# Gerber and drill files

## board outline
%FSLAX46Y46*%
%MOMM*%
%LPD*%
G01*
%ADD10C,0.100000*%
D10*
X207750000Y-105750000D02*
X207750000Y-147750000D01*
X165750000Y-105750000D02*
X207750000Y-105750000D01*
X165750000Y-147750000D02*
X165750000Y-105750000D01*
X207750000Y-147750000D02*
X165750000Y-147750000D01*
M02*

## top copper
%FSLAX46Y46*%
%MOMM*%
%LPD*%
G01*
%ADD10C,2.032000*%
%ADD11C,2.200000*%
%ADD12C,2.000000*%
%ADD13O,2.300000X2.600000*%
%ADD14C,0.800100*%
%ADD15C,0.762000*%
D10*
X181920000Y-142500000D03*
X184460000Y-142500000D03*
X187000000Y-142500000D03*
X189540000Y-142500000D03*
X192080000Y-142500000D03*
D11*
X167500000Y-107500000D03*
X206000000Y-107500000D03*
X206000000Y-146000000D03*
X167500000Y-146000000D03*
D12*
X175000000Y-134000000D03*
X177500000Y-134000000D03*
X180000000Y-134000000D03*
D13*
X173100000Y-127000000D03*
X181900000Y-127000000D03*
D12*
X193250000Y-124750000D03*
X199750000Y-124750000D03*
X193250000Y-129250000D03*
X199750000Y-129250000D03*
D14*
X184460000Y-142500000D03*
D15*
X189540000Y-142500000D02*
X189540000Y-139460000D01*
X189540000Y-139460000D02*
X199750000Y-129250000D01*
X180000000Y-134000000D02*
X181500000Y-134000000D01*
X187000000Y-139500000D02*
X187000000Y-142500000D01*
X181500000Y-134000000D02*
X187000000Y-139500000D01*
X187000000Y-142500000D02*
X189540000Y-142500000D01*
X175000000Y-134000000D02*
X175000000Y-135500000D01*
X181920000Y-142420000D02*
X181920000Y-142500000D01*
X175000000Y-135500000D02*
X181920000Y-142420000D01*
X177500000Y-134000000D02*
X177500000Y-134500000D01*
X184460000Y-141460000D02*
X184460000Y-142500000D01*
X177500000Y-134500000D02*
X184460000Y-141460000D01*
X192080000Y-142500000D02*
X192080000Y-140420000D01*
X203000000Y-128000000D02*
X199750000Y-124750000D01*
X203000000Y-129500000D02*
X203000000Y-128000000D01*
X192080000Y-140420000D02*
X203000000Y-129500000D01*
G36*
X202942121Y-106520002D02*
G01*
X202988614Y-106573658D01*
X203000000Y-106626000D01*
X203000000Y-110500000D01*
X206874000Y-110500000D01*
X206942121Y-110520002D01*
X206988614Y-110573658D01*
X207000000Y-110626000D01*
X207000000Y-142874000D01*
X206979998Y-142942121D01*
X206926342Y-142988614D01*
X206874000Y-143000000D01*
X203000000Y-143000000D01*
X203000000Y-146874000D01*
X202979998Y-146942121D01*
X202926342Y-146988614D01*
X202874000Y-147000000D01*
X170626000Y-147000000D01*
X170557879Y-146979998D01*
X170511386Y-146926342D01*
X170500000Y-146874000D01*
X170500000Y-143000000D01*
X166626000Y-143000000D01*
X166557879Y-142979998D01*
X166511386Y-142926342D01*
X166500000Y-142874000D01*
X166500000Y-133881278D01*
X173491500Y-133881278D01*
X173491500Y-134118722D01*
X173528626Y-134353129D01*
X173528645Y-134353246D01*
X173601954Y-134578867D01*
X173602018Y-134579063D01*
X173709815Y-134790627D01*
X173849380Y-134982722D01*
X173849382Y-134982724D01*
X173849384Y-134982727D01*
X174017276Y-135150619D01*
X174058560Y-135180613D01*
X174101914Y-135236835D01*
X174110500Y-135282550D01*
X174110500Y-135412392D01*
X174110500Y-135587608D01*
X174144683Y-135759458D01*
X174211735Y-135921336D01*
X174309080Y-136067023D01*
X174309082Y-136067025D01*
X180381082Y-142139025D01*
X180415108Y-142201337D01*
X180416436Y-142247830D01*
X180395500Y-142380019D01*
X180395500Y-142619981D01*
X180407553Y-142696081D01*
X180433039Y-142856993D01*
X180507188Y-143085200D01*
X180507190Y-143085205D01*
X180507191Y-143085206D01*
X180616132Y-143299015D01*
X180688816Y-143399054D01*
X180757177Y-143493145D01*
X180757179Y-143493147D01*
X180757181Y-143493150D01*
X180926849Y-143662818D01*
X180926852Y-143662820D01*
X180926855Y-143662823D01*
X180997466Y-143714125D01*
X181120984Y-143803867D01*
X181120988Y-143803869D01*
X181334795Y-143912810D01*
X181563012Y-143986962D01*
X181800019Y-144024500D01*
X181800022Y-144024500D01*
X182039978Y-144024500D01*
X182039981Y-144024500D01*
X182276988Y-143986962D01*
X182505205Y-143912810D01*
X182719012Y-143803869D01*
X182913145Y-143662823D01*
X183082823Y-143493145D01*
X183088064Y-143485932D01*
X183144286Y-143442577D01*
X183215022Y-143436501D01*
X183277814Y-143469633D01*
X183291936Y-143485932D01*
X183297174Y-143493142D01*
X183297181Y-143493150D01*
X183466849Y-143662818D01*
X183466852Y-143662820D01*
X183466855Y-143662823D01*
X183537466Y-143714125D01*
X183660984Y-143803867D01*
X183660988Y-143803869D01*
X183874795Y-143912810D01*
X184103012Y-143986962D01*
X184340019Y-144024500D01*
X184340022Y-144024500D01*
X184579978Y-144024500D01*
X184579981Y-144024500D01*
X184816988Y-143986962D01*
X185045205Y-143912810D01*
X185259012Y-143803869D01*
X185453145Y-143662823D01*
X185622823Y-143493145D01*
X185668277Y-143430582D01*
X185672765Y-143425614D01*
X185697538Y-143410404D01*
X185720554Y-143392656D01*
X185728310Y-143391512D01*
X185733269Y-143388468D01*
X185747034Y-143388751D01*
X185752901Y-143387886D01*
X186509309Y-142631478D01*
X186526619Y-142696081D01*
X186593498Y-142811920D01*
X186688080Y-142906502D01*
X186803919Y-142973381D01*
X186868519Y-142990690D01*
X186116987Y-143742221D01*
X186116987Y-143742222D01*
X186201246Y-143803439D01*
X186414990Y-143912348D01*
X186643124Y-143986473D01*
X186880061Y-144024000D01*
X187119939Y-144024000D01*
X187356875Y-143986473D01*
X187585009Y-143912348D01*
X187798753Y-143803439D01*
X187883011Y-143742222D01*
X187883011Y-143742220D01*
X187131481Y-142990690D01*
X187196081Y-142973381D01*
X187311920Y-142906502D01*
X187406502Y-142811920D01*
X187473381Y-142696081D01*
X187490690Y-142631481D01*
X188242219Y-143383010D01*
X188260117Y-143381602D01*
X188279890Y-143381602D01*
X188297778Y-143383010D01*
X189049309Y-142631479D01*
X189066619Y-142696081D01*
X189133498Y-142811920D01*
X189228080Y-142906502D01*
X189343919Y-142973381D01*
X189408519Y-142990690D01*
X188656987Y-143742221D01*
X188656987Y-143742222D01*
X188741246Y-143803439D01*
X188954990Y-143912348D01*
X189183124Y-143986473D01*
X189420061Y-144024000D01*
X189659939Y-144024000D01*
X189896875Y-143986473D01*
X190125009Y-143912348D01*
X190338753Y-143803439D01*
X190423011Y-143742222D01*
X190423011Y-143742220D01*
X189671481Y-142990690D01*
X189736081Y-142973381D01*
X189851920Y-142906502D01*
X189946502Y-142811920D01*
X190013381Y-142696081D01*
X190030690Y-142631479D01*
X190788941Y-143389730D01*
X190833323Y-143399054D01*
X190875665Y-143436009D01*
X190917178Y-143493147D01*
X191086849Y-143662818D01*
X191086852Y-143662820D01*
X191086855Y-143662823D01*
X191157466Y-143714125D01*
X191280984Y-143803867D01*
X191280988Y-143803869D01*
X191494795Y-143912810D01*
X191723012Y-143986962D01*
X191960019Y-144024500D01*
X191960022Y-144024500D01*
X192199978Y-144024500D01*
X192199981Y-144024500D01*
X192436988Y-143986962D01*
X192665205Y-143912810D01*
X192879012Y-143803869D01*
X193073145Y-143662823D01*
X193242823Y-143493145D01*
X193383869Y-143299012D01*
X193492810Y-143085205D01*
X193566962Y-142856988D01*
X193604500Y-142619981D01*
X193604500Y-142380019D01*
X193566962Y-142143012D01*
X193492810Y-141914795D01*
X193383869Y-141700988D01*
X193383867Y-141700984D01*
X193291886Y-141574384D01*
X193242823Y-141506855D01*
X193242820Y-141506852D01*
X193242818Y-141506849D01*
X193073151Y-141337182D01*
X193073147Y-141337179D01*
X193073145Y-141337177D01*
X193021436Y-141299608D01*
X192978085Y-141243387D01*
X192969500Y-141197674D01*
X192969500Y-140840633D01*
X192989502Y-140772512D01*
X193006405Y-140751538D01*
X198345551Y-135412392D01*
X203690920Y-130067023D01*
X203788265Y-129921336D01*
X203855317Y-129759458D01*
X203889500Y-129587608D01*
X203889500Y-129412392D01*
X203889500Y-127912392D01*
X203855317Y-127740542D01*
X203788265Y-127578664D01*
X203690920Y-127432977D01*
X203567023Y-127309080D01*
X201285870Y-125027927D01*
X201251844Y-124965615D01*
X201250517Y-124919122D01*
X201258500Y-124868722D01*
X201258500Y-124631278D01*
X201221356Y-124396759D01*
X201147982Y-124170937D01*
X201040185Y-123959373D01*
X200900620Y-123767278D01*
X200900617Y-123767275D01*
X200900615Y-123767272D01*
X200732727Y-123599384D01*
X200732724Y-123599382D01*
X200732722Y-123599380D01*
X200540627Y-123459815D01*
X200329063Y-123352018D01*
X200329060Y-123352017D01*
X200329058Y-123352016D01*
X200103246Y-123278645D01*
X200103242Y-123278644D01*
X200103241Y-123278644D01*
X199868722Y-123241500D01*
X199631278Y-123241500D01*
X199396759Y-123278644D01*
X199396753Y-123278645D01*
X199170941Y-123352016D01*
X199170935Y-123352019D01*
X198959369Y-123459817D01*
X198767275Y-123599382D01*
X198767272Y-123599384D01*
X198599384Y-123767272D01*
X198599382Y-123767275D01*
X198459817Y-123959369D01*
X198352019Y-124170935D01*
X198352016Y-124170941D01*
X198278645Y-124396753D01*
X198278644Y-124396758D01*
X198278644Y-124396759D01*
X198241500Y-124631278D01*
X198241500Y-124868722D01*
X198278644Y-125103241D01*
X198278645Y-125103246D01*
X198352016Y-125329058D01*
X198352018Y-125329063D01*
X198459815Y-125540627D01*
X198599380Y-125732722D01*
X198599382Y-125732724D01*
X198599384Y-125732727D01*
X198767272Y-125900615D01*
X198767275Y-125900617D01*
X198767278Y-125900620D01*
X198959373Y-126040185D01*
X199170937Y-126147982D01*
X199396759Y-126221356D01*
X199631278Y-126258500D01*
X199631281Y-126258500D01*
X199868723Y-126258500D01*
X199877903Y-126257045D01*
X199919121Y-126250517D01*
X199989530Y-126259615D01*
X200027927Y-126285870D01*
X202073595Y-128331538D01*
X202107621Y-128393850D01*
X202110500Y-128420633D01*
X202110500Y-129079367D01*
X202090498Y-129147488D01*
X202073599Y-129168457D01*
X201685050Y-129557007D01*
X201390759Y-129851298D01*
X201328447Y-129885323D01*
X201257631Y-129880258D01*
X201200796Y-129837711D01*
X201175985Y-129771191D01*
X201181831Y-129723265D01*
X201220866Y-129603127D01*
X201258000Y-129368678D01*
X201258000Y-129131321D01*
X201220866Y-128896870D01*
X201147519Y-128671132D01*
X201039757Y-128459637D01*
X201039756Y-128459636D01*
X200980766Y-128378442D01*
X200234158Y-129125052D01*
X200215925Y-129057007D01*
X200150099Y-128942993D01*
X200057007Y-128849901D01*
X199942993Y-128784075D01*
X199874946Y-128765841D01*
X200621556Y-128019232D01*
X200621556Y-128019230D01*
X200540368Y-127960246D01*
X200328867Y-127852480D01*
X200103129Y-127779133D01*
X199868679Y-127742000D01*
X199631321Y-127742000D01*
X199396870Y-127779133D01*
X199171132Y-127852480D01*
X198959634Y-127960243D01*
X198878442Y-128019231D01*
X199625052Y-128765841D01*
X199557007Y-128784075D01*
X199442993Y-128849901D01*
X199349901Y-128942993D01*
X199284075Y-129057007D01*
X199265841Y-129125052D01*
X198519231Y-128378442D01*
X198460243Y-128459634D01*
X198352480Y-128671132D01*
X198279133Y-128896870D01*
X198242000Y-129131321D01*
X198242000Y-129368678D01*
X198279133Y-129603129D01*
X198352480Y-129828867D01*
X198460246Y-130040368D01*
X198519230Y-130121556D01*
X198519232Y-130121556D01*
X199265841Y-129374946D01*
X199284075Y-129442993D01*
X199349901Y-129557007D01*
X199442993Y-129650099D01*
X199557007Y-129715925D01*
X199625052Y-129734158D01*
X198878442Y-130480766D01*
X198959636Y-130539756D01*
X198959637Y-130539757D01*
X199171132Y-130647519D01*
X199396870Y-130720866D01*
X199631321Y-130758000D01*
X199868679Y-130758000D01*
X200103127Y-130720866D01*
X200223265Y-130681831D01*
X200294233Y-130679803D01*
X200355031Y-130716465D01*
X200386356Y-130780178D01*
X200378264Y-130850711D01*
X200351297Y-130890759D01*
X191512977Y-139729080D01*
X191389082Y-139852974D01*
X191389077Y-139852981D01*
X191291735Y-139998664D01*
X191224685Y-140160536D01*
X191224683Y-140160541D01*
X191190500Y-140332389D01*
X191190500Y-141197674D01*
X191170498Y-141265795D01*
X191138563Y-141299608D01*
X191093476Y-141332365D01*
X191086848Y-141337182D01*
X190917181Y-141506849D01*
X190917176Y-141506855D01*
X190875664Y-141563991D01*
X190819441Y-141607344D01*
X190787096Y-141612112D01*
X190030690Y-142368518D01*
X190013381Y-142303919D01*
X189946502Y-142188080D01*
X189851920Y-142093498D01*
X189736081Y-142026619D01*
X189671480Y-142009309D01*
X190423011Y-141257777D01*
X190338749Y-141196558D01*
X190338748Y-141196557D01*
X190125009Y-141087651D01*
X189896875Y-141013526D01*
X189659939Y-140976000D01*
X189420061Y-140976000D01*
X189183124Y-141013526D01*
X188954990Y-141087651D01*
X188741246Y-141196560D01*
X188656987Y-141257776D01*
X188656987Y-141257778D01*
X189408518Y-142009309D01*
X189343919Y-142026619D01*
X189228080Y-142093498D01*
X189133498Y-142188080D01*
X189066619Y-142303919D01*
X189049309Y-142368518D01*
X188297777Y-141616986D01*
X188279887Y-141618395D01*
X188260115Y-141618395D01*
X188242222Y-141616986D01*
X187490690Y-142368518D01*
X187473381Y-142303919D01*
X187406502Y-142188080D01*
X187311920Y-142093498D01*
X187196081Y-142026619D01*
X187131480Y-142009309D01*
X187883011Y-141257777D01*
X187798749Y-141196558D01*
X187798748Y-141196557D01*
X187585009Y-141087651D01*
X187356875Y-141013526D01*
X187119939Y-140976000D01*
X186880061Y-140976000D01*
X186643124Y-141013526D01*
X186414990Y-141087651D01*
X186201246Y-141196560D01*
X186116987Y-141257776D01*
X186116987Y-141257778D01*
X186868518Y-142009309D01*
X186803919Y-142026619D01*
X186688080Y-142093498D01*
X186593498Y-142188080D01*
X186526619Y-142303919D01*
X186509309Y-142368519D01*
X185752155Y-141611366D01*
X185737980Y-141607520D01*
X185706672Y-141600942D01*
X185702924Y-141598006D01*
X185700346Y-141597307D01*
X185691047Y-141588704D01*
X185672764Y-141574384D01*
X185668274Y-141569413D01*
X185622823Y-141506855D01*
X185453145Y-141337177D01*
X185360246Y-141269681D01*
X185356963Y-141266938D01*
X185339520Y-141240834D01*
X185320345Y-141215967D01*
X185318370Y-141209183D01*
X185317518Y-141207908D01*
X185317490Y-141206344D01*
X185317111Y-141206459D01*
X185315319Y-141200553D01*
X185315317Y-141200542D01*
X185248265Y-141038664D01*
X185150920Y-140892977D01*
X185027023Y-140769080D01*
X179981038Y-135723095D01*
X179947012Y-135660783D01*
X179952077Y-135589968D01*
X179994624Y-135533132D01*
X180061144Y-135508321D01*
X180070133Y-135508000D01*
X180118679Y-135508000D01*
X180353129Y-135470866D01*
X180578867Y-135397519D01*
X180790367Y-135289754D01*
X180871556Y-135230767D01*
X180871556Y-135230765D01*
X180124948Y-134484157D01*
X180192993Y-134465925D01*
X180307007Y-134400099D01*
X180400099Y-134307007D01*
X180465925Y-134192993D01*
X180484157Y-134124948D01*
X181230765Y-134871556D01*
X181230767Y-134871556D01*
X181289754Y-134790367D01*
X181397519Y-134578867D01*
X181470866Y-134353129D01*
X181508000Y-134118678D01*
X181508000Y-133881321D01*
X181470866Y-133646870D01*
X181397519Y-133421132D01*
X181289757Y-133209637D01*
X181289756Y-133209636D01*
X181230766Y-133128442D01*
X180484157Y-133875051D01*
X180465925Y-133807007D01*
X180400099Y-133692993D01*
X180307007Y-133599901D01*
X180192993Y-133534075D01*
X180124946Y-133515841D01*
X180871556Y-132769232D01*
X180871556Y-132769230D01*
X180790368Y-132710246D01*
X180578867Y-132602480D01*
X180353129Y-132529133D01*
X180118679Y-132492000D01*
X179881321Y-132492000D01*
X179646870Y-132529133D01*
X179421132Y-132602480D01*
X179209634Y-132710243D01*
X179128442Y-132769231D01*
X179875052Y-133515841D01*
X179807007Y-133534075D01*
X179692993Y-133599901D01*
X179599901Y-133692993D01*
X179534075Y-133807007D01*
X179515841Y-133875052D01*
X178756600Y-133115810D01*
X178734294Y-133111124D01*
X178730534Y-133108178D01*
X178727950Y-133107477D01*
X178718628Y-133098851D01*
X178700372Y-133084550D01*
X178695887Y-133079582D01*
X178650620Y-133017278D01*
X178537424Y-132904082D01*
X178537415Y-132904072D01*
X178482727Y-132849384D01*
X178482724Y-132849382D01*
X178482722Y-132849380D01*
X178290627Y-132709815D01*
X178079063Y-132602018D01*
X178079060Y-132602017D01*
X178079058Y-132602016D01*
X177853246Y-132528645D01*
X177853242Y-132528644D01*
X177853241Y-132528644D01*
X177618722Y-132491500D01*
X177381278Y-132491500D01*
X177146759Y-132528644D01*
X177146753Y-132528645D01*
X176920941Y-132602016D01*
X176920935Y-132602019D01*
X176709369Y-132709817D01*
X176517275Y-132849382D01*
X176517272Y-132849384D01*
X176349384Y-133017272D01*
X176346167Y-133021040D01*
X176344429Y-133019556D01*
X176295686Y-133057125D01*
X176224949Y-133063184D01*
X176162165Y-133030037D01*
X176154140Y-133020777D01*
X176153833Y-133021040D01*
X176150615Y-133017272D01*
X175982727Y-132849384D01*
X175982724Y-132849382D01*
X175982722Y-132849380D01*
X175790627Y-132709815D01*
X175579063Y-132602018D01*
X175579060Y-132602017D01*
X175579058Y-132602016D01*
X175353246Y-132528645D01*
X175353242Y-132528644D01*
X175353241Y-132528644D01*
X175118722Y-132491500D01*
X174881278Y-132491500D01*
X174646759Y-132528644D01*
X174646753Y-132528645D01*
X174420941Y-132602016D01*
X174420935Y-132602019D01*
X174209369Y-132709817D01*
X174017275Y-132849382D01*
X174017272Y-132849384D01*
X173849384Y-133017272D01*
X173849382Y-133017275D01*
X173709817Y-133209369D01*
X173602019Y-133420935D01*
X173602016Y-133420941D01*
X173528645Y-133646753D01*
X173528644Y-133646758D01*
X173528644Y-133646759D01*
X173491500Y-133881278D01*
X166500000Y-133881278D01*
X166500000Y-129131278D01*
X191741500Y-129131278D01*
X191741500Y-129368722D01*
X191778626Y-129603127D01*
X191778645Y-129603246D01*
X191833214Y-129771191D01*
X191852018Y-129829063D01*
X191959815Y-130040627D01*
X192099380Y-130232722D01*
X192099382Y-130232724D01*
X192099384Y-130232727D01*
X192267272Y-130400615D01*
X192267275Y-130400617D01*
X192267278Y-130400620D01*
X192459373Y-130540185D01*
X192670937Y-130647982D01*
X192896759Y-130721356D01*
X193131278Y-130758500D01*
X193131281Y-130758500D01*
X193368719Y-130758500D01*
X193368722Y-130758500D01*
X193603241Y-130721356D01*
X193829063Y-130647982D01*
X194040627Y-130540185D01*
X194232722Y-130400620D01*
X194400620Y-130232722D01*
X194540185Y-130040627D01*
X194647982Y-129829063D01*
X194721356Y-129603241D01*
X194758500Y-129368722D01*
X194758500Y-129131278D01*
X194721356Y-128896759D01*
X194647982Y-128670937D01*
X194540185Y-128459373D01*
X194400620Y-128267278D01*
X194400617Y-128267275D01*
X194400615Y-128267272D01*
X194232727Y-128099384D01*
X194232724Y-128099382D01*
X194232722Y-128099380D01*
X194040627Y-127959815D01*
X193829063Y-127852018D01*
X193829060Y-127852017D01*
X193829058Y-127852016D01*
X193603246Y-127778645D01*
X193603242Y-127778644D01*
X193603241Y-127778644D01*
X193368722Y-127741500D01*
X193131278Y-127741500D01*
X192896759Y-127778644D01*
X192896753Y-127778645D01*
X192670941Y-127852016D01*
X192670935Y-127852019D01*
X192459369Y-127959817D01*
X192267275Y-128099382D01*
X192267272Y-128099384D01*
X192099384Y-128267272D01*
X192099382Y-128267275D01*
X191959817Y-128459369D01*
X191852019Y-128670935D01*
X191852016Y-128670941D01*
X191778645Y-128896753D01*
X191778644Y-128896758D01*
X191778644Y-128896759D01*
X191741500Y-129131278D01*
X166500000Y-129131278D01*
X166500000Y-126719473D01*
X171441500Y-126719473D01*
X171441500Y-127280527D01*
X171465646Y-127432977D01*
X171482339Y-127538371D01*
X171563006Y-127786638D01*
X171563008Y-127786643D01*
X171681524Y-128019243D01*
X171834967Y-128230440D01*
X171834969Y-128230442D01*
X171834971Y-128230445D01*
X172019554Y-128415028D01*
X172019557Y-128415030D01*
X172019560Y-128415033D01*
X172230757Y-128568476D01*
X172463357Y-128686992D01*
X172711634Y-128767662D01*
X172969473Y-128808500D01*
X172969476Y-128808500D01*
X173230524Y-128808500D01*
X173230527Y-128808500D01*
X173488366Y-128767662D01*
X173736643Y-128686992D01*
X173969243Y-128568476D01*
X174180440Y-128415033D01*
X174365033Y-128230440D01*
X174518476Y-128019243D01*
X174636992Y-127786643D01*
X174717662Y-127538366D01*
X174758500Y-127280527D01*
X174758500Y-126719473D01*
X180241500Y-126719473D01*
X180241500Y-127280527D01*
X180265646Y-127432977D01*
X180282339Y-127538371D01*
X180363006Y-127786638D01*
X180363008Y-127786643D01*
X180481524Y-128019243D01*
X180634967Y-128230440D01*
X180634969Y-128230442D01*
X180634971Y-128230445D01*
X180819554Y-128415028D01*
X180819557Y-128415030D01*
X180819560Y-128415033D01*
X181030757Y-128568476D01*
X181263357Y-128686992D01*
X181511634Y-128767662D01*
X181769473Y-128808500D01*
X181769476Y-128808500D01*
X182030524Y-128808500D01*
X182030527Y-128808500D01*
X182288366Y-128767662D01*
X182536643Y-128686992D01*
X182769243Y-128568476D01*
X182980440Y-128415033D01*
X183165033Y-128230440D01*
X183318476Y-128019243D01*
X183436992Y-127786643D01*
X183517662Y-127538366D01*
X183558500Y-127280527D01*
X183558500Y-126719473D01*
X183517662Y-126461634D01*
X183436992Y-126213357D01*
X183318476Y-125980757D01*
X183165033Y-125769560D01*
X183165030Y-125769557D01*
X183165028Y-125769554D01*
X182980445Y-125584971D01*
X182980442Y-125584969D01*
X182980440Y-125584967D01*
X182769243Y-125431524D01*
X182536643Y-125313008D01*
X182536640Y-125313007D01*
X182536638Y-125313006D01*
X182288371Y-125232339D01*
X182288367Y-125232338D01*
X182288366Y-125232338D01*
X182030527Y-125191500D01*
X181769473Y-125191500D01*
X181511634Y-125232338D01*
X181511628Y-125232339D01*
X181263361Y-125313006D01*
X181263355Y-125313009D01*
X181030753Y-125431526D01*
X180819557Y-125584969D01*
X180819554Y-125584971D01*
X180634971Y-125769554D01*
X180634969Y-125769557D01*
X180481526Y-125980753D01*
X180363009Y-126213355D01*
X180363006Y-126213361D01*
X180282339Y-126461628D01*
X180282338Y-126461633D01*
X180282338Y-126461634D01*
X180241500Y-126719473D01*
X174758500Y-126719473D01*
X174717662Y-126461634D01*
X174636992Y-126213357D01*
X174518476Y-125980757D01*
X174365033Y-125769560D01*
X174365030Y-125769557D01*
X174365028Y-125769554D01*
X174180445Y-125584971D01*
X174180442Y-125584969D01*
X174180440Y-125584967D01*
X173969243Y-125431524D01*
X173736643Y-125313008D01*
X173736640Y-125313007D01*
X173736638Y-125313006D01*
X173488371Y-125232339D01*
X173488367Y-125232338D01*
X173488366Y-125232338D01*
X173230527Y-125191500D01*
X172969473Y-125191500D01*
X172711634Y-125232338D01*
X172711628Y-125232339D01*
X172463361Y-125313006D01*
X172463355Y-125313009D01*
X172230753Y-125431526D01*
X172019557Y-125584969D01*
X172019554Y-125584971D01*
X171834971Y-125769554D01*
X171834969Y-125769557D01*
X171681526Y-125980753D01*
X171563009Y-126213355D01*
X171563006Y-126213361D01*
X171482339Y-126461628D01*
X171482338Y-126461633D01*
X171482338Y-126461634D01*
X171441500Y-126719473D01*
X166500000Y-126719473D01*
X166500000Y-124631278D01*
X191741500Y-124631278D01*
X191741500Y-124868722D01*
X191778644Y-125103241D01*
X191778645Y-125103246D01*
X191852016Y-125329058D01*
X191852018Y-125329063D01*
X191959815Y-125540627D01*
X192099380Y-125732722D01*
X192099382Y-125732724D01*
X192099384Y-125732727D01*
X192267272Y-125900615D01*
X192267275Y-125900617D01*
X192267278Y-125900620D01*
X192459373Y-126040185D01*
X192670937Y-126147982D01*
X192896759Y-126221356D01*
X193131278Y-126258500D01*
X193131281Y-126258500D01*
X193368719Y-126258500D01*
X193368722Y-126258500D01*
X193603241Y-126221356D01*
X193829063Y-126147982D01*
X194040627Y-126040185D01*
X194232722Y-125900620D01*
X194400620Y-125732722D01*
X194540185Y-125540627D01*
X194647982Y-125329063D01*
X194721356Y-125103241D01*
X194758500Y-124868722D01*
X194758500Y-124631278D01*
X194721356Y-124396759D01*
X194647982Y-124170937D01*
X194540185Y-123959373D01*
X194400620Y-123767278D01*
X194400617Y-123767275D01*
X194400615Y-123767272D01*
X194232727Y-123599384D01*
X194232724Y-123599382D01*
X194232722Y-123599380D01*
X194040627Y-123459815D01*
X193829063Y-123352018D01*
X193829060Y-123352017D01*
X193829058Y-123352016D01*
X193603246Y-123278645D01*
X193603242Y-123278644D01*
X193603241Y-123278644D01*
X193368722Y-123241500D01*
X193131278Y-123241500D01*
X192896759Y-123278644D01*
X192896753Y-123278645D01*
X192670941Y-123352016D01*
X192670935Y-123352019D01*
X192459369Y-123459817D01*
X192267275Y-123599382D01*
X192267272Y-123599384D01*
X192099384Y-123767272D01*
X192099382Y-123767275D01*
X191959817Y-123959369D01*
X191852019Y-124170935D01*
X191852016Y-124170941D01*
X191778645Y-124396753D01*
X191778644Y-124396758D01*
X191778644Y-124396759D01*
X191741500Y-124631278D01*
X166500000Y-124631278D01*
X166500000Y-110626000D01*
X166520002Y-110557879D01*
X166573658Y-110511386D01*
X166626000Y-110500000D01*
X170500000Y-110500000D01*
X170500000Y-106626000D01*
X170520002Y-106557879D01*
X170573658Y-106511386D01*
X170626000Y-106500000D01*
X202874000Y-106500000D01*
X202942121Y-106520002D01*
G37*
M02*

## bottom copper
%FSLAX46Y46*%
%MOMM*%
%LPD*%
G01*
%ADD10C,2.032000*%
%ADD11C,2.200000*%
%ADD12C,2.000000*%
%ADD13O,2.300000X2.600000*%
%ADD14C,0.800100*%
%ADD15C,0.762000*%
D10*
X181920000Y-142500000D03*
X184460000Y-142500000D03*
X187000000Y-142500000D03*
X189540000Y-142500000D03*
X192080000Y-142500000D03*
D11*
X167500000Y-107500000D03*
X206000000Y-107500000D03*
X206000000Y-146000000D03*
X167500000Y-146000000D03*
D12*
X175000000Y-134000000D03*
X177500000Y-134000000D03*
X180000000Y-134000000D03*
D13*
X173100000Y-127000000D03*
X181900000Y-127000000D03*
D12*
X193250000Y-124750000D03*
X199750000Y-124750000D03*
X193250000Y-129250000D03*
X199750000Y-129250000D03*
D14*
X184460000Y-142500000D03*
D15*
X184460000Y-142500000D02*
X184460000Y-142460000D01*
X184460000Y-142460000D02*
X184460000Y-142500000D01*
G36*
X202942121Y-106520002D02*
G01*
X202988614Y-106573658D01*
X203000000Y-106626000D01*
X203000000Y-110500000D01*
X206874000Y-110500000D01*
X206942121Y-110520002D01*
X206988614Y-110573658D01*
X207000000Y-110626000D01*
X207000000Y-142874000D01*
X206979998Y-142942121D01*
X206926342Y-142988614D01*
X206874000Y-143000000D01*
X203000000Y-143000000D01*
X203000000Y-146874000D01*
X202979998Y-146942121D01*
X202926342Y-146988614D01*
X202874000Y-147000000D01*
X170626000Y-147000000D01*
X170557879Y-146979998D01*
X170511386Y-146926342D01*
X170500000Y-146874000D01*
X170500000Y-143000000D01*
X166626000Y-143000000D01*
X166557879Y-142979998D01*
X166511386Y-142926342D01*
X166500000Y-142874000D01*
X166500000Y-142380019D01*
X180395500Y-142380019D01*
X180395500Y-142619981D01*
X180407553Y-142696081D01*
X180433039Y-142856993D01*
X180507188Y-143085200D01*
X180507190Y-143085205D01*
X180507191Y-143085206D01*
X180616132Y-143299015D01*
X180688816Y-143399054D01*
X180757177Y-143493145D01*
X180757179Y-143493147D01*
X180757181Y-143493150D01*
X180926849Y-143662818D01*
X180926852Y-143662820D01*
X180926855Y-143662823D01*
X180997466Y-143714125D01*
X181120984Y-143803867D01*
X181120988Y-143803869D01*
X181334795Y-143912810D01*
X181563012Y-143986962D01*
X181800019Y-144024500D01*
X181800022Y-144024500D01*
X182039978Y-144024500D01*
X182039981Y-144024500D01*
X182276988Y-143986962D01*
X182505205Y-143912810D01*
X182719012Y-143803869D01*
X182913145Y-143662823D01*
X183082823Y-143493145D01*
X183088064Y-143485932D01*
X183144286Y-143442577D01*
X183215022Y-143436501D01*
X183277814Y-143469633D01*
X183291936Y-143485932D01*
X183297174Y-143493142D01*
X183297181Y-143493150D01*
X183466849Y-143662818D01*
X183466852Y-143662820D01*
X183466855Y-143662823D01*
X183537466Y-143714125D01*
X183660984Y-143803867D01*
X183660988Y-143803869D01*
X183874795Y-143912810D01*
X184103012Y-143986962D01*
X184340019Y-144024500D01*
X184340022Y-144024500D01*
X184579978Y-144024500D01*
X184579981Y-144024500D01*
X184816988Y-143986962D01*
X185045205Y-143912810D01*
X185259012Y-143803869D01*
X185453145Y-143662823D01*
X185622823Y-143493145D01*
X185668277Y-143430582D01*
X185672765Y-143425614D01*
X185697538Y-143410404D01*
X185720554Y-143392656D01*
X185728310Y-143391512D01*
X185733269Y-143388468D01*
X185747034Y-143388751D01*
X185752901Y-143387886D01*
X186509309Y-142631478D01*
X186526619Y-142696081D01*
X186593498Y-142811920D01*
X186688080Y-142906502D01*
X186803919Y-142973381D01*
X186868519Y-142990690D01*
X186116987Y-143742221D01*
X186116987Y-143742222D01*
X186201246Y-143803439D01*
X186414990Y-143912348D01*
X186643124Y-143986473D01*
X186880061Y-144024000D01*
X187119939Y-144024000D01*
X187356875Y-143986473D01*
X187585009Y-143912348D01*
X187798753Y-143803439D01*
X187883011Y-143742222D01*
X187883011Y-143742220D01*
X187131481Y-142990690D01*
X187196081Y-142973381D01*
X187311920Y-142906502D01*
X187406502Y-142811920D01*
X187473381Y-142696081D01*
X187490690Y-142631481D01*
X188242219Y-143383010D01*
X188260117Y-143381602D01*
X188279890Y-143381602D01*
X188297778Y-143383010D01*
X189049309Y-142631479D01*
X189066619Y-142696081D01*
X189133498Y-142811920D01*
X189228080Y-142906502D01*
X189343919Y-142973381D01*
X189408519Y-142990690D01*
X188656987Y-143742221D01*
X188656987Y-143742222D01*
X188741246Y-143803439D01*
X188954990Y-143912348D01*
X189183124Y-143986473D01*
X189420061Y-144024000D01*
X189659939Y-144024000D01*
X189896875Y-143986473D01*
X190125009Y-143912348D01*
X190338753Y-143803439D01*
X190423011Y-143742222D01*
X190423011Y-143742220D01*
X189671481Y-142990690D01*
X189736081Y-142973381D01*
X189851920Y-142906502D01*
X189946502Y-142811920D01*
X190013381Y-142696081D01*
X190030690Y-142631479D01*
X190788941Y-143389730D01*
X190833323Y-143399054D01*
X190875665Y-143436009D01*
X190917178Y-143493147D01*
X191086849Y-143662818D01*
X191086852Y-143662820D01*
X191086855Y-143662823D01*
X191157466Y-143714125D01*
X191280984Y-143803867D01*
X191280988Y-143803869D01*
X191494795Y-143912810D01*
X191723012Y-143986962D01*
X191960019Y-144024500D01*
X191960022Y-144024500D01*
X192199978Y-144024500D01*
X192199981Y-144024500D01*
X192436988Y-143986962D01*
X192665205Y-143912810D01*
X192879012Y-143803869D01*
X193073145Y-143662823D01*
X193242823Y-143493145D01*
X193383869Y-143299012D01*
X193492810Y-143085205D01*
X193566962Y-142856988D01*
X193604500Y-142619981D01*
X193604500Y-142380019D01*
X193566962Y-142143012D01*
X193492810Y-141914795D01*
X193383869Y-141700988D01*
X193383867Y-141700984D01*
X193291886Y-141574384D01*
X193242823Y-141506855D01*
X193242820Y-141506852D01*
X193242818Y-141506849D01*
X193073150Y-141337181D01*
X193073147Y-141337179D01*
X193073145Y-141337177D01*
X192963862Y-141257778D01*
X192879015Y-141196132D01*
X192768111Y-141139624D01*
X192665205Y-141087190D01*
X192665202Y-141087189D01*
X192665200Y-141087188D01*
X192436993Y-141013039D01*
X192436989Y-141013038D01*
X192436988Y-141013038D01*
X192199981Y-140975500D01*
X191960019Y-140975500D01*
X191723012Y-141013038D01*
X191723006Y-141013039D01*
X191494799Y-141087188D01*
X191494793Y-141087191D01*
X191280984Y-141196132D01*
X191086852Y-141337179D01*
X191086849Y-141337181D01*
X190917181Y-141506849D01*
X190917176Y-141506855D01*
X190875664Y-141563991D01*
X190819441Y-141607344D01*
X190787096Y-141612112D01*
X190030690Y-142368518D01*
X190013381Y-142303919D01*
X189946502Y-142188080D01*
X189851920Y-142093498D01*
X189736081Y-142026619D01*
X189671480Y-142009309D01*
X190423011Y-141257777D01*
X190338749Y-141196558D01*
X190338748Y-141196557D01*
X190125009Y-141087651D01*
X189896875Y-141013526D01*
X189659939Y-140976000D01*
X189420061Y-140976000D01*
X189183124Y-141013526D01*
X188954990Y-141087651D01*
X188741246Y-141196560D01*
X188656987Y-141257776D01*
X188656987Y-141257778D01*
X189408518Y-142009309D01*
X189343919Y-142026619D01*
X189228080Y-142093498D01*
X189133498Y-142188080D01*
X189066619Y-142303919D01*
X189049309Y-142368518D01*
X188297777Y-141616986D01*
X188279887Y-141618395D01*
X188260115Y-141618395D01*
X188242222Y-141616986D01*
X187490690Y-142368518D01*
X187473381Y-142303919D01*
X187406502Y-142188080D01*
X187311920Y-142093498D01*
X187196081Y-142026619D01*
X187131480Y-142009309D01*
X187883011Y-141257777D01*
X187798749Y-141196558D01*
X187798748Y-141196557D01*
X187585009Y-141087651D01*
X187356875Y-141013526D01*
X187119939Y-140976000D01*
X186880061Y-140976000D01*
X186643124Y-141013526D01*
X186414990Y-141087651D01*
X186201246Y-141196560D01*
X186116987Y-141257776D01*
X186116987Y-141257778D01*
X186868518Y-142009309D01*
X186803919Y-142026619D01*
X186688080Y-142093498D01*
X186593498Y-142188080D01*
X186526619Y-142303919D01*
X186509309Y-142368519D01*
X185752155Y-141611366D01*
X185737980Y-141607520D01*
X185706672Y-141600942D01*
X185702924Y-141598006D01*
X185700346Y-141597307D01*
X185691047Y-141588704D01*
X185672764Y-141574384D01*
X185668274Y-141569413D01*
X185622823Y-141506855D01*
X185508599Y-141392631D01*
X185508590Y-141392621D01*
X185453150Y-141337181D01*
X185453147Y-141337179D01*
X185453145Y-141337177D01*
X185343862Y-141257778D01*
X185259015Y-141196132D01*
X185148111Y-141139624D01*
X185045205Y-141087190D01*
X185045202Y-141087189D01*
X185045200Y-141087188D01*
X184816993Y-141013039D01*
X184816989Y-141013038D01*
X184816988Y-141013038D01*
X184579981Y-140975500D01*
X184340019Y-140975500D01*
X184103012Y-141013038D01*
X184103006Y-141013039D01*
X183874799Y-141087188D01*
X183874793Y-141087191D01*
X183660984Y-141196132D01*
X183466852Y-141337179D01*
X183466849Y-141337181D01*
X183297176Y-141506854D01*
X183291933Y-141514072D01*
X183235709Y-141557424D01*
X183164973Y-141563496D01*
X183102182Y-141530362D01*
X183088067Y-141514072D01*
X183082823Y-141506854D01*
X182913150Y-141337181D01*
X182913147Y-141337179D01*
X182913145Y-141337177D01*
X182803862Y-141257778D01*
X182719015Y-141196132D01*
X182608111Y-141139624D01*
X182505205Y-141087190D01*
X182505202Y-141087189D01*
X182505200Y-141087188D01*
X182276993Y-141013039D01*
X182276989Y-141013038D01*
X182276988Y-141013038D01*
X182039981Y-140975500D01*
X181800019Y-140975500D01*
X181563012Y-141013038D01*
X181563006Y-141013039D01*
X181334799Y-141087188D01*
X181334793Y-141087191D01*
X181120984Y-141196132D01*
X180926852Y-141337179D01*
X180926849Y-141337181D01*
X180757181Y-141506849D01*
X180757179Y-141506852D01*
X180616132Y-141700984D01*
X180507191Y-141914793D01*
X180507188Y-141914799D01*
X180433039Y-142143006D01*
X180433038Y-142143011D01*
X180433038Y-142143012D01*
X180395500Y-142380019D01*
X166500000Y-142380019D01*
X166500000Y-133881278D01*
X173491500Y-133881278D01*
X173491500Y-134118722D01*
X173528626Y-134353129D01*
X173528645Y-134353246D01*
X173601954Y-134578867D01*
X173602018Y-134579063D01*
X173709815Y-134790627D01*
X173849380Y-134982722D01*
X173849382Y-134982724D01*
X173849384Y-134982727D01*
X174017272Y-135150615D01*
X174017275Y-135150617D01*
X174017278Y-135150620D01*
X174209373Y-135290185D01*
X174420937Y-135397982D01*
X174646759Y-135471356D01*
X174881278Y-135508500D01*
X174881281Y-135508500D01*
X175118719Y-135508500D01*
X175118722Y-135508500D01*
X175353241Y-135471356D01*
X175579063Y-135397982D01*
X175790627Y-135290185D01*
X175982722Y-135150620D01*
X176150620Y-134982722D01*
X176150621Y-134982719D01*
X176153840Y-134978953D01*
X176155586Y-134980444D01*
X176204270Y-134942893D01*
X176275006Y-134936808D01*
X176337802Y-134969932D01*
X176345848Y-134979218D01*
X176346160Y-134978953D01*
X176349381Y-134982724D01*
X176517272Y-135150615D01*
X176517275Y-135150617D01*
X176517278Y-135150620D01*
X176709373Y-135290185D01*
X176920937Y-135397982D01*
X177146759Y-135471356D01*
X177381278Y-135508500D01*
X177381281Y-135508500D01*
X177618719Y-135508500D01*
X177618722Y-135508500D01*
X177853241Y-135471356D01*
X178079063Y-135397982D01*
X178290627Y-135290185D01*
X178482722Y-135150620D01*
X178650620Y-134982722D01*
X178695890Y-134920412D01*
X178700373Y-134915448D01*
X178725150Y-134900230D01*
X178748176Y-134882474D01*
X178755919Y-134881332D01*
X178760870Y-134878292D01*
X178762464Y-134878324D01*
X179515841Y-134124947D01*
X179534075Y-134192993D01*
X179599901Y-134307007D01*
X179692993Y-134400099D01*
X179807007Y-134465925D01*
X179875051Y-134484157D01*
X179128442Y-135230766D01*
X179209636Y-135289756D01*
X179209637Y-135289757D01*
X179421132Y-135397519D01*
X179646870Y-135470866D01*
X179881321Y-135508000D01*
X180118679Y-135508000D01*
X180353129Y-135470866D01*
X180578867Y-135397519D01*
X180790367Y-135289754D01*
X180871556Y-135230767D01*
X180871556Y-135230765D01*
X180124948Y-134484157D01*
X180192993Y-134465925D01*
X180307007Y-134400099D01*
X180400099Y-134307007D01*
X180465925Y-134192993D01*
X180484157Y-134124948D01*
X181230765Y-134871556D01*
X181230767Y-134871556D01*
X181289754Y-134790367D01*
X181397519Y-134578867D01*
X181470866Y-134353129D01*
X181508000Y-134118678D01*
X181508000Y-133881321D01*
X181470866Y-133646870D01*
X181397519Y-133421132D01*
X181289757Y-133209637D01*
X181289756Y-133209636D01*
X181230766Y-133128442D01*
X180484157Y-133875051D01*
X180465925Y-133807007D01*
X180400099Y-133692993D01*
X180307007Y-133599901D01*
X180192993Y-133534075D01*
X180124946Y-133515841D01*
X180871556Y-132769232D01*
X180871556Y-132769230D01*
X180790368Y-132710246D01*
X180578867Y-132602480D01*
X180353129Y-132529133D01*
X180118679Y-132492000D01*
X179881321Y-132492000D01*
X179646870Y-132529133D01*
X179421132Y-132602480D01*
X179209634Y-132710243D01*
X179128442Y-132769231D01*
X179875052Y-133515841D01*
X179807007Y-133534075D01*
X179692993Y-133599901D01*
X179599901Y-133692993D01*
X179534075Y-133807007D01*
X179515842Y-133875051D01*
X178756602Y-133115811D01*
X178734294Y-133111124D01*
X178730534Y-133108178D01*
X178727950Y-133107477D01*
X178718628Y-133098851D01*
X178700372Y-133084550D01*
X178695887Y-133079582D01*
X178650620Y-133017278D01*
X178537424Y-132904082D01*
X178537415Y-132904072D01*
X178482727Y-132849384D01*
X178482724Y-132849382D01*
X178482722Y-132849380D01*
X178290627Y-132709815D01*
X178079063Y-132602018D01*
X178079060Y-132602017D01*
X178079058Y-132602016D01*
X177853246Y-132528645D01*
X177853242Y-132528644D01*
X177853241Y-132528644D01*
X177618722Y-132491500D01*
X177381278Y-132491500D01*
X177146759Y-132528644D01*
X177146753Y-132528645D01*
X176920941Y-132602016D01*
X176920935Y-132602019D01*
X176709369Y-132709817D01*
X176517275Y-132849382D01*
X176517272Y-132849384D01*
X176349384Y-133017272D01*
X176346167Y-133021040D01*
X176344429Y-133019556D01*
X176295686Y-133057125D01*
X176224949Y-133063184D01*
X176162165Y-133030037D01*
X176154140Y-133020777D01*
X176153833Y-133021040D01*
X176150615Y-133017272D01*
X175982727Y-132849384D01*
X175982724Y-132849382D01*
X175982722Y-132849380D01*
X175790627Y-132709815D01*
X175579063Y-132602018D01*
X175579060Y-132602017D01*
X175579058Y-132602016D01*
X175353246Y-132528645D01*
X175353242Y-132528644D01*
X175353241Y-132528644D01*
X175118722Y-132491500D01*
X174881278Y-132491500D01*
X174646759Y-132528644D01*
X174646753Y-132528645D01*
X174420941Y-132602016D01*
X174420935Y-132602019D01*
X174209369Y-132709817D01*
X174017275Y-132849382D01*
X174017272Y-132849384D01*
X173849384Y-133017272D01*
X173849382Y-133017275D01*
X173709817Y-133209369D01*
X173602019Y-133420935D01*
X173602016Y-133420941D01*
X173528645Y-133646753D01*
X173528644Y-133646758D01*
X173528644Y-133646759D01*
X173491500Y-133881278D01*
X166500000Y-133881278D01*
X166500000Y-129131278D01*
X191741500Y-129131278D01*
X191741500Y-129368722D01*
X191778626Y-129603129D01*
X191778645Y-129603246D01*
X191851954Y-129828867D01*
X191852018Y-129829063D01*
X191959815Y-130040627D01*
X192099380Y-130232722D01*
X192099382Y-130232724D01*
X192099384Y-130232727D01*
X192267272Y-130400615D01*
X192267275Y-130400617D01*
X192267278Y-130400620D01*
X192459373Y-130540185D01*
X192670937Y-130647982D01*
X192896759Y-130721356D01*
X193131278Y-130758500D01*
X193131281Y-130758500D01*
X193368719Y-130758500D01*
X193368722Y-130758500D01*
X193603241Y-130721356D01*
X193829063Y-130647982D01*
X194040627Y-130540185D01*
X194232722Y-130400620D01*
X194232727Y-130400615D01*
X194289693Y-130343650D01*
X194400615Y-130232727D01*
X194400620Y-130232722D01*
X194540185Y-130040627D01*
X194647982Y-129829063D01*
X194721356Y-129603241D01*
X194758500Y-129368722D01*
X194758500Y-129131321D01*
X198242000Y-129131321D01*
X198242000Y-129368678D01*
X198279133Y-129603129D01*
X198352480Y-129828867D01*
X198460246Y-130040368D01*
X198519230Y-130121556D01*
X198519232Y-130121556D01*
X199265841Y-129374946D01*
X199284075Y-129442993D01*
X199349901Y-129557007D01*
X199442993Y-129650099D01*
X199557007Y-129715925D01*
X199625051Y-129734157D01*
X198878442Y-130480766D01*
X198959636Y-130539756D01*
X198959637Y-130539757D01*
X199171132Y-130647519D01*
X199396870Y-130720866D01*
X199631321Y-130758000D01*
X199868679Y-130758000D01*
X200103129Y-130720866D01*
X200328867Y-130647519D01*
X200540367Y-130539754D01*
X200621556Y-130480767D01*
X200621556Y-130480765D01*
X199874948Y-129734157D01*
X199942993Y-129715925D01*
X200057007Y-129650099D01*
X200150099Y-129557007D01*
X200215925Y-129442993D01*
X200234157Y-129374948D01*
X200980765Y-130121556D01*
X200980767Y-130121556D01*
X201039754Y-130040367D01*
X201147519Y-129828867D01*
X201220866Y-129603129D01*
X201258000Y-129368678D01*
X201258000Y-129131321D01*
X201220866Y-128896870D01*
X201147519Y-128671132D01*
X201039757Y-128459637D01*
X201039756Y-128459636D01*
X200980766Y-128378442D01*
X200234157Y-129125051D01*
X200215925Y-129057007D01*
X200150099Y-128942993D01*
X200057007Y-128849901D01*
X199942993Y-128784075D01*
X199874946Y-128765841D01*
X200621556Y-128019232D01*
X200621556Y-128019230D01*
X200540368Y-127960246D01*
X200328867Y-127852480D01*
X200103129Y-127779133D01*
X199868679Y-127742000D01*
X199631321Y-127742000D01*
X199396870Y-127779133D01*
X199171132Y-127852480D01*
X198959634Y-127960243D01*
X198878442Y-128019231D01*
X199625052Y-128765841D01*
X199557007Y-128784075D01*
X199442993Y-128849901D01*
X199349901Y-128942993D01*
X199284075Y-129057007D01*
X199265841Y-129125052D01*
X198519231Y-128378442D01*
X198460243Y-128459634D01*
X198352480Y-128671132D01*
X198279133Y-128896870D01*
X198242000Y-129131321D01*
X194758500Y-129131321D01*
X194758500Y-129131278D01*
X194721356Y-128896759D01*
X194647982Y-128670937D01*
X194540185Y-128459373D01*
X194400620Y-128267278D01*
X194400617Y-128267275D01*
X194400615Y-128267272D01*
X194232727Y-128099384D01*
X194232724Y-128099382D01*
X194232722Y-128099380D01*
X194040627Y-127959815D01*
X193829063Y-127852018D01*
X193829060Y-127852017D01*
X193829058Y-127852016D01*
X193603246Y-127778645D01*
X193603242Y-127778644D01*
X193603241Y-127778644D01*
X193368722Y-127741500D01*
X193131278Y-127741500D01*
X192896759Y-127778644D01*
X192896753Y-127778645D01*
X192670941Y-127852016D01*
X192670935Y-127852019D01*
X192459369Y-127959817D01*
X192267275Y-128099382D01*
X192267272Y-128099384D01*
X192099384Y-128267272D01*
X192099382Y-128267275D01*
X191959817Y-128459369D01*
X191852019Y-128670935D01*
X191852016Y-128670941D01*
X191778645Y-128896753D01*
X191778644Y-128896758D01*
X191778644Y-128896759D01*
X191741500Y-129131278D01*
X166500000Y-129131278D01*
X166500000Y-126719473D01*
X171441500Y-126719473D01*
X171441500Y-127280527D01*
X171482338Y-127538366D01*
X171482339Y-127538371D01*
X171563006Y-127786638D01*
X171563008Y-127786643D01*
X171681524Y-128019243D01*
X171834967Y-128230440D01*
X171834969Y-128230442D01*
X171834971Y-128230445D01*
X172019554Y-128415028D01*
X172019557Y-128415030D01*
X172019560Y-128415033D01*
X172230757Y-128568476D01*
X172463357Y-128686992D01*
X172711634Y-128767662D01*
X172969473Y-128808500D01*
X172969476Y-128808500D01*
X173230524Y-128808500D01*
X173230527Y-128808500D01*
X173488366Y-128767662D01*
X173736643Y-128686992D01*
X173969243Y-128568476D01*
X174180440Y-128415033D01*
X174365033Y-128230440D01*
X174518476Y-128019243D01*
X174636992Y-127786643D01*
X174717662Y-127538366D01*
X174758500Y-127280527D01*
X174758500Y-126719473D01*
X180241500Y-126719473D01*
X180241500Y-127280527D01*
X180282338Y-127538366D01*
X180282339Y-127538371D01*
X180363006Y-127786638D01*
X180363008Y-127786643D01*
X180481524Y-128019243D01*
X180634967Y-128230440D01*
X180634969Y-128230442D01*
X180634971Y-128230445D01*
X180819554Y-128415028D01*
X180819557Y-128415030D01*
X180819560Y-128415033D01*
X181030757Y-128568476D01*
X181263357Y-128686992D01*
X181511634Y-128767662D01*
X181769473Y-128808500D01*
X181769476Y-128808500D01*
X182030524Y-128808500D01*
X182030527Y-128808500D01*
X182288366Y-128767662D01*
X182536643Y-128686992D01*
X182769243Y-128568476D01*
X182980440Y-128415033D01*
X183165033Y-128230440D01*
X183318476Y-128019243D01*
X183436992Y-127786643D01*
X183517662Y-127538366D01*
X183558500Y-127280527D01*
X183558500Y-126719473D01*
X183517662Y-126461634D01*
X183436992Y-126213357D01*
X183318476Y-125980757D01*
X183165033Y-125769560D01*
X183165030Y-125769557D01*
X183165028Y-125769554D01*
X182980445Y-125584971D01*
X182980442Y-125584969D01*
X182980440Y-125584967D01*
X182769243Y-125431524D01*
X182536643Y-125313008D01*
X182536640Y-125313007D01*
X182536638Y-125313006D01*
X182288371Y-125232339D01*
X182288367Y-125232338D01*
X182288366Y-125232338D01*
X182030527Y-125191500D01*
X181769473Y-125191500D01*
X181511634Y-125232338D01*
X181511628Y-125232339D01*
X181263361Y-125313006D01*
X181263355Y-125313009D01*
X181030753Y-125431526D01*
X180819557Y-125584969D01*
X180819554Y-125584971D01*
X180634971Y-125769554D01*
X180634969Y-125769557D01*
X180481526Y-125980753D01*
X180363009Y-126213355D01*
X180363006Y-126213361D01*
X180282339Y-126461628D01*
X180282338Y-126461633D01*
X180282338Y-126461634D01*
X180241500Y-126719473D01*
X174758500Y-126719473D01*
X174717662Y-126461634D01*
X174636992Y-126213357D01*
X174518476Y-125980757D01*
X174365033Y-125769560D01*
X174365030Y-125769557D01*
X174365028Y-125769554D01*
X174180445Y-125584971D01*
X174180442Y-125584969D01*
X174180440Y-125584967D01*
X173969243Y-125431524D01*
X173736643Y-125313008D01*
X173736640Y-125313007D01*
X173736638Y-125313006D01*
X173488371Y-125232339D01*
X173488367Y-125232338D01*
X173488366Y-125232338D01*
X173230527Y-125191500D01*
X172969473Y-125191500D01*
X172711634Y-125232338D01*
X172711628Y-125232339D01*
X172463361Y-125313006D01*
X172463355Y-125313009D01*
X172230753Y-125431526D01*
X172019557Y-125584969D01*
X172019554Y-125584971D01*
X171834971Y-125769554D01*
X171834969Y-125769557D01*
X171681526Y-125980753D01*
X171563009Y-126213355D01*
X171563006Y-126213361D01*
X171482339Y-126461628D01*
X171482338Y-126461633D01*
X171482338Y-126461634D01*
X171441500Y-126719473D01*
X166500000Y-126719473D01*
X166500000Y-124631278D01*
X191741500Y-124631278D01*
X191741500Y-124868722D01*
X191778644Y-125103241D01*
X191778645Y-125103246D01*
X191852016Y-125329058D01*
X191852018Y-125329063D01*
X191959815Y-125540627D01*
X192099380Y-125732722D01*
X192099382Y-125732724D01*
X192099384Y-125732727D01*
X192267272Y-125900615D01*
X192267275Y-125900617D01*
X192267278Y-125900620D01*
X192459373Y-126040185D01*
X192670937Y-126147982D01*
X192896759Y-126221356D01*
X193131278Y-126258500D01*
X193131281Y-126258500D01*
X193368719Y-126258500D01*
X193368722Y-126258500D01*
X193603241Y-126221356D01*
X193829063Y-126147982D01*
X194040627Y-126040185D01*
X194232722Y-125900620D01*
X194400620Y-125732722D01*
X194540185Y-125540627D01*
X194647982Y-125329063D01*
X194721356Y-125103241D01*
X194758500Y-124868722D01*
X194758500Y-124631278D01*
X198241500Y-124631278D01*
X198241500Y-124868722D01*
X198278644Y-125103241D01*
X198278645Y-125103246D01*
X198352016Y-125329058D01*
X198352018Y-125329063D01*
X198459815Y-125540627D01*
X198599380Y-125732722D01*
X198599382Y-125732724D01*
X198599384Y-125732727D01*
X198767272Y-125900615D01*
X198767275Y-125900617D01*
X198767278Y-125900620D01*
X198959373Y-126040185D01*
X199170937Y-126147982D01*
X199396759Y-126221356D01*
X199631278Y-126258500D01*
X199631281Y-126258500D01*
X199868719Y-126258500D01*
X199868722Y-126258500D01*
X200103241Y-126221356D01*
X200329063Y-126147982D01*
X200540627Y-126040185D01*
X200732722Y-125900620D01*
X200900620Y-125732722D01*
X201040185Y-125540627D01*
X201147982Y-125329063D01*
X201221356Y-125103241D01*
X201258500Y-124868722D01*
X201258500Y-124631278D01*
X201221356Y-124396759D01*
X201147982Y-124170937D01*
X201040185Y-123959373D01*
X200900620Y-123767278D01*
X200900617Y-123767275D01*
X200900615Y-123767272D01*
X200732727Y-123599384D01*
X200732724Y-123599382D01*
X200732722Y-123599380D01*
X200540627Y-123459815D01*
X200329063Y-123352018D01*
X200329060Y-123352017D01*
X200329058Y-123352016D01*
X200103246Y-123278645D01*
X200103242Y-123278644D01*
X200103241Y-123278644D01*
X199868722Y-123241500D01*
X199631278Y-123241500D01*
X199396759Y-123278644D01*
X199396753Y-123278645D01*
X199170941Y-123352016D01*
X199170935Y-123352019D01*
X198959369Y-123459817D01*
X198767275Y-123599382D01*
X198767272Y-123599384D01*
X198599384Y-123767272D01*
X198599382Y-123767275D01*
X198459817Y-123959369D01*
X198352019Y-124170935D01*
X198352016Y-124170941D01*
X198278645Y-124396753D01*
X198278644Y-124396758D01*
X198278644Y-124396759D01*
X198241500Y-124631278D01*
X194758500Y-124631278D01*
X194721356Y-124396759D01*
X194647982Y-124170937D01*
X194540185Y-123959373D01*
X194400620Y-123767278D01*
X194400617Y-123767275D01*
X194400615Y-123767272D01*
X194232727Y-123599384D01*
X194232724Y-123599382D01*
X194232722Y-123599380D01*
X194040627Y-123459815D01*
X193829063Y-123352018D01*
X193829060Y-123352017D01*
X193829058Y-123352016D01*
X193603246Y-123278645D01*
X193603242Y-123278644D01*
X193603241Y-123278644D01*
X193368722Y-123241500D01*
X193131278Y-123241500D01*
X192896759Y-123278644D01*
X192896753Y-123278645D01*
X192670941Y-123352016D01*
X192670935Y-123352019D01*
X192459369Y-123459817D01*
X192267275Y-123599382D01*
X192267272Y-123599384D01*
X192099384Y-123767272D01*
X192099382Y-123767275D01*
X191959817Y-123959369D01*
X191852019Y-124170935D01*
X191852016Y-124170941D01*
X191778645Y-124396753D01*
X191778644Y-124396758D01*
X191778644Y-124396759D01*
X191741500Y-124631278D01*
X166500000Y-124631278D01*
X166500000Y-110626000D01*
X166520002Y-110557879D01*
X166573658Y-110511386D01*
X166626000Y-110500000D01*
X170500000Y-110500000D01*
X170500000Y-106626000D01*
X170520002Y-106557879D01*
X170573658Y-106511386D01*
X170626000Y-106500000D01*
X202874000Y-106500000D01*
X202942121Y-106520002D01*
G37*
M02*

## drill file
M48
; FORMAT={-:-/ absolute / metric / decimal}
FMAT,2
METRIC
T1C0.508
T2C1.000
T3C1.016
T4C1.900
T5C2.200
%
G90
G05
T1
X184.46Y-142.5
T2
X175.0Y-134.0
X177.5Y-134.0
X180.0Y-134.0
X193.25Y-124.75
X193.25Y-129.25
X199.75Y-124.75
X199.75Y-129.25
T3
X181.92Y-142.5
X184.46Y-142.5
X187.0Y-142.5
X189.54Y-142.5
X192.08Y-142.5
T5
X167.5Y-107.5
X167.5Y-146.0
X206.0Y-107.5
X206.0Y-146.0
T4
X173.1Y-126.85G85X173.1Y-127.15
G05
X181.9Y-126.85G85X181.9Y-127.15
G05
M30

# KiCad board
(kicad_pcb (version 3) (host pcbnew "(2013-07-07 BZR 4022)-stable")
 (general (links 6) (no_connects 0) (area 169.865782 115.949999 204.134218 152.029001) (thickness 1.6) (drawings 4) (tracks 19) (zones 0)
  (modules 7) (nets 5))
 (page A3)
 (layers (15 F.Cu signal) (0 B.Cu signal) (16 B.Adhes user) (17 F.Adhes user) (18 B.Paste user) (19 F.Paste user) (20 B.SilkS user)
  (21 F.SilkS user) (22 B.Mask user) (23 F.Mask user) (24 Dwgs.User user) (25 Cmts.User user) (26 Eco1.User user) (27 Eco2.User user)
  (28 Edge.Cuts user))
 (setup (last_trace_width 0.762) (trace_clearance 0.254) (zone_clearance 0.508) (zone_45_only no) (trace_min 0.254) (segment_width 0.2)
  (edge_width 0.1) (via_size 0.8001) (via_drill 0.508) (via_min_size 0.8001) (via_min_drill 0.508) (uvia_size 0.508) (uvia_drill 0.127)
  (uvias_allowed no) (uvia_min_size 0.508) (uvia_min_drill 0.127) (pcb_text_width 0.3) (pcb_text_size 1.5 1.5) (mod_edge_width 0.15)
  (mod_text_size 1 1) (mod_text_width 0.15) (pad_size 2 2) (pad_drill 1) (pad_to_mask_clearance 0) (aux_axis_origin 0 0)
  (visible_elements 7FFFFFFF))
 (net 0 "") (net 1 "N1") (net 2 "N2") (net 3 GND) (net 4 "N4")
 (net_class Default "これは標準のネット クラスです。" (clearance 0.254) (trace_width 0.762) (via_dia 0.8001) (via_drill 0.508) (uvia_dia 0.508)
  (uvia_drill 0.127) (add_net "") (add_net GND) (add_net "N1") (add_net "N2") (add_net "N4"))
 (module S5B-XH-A (layer B.Cu) (at 187 142.5)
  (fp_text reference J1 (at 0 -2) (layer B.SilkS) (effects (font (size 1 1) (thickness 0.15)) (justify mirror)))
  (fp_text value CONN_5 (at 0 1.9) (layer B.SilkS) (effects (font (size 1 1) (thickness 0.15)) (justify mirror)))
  (pad 1 thru_hole circle (at -5.08 0) (size 2.032 2.032) (drill 1.016) (layers *.Cu *.Mask B.SilkS) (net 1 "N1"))
  (pad 2 thru_hole circle (at -2.54 0) (size 2.032 2.032) (drill 1.016) (layers *.Cu *.Mask B.SilkS) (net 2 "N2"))
  (pad 3 thru_hole circle (at 0 0) (size 2.032 2.032) (drill 1.016) (layers *.Cu *.Mask B.SilkS) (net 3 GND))
  (pad 4 thru_hole circle (at 2.54 0) (size 2.032 2.032) (drill 1.016) (layers *.Cu *.Mask B.SilkS) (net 3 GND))
  (pad 5 thru_hole circle (at 5.08 0) (size 2.032 2.032) (drill 1.016) (layers *.Cu *.Mask B.SilkS) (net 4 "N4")))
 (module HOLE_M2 (layer F.Cu) (at 167.5 107.5)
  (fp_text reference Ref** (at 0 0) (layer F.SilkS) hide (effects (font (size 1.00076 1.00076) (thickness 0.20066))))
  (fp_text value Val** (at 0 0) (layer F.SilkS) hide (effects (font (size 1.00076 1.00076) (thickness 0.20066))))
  (pad "" thru_hole circle (at 0 0) (size 2.2 2.2) (drill 2.2) (layers *.Cu *.Mask F.SilkS) (clearance 1.50114)))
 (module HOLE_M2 (layer F.Cu) (at 206 107.5)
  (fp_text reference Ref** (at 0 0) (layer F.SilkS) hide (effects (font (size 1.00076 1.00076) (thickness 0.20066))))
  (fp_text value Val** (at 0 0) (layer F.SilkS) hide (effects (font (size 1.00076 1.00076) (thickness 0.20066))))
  (pad "" thru_hole circle (at 0 0) (size 2.2 2.2) (drill 2.2) (layers *.Cu *.Mask F.SilkS) (clearance 1.50114)))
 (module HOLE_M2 (layer F.Cu) (at 206 146)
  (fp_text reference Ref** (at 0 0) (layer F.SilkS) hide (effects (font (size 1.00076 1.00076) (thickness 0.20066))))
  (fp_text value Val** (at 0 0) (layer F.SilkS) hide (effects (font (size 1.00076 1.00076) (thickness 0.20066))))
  (pad "" thru_hole circle (at 0 0) (size 2.2 2.2) (drill 2.2) (layers *.Cu *.Mask F.SilkS) (clearance 1.50114)))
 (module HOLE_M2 (layer F.Cu) (at 167.5 146)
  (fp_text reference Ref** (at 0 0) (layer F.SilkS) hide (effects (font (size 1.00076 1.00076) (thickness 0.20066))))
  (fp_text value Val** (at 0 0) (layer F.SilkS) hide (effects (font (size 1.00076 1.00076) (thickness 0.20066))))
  (pad "" thru_hole circle (at 0 0) (size 2.2 2.2) (drill 2.2) (layers *.Cu *.Mask F.SilkS) (clearance 1.50114)))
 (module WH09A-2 (layer F.Cu) (at 177.5 127)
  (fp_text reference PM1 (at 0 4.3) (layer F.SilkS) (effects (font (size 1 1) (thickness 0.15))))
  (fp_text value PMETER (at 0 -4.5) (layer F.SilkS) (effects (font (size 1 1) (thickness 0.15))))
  (pad 1 thru_hole circle (at -2.5 7) (size 2 2) (drill 1) (layers *.Cu *.Mask F.SilkS) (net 1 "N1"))
  (pad 2 thru_hole circle (at 0 7) (size 2 2) (drill 1) (layers *.Cu *.Mask F.SilkS) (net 2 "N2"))
  (pad 3 thru_hole circle (at 2.5 7) (size 2 2) (drill 1) (layers *.Cu *.Mask F.SilkS) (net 3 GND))
  (pad "" thru_hole oval (at -4.4 0) (size 2.3 2.6) (drill oval 1.9 2.2) (layers *.Cu *.Mask F.SilkS))
  (pad "" thru_hole oval (at 4.4 0) (size 2.3 2.6) (drill oval 1.9 2.2) (layers *.Cu *.Mask F.SilkS)))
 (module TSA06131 (layer F.Cu) (at 196.5 127)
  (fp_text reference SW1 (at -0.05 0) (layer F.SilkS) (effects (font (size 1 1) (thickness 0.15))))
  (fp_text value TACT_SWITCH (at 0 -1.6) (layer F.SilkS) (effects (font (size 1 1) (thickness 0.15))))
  (pad 4 thru_hole circle (at -3.25 -2.25) (size 2 2) (drill 1) (layers *.Cu *.Mask F.SilkS))
  (pad 1 thru_hole circle (at 3.25 -2.25) (size 2 2) (drill 1) (layers *.Cu *.Mask F.SilkS) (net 4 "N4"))
  (pad 3 thru_hole circle (at -3.25 2.25) (size 2 2) (drill 1) (layers *.Cu *.Mask F.SilkS))
  (pad 2 thru_hole circle (at 3.25 2.25) (size 2 2) (drill 1) (layers *.Cu *.Mask F.SilkS) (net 3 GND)))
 (gr_line (start 207.75 105.75) (end 207.75 147.75) (angle 90) (layer Edge.Cuts) (width 0.1))
 (gr_line (start 165.75 105.75) (end 207.75 105.75) (angle 90) (layer Edge.Cuts) (width 0.1))
 (gr_line (start 165.75 147.75) (end 165.75 105.75) (angle 90) (layer Edge.Cuts) (width 0.1))
 (gr_line (start 207.75 147.75) (end 165.75 147.75) (angle 90) (layer Edge.Cuts) (width 0.1))
 (segment (start 189.54 142.5) (end 189.54 139.46) (width 0.762) (layer F.Cu) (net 3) (status 400000))
 (segment (start 189.54 139.46) (end 199.75 129.25) (width 0.762) (layer F.Cu) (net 3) (status 800000))
 (segment (start 180 134) (end 181.5 134) (width 0.762) (layer F.Cu) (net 3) (status 400000))
 (segment (start 187 139.5) (end 187 142.5) (width 0.762) (layer F.Cu) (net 3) (status 800000))
 (segment (start 181.5 134) (end 187 139.5) (width 0.762) (layer F.Cu) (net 3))
 (segment (start 187 142.5) (end 189.54 142.5) (width 0.762) (layer F.Cu) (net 3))
 (segment (start 175 134) (end 175 135.5) (width 0.762) (layer F.Cu) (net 1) (status 400000))
 (segment (start 181.92 142.42) (end 181.92 142.5) (width 0.762) (layer F.Cu) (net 1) (status C00000))
 (segment (start 175 135.5) (end 181.92 142.42) (width 0.762) (layer F.Cu) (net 1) (status 800000))
 (segment (start 177.5 134) (end 177.5 134.5) (width 0.762) (layer F.Cu) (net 2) (status C00000))
 (segment (start 184.46 141.46) (end 184.46 142.5) (width 0.762) (layer F.Cu) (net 2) (status 800000))
 (segment (start 177.5 134.5) (end 184.46 141.46) (width 0.762) (layer F.Cu) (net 2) (status 400000))
 (segment (start 184.46 142.5) (end 184.46 142.46) (width 0.762) (layer B.Cu) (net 2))
 (segment (start 184.46 142.46) (end 184.46 142.5) (width 0.762) (layer B.Cu) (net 2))
 (via (at 184.46 142.5) (size 0.8001) (layers F.Cu B.Cu) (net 2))
 (segment (start 192.08 142.5) (end 192.08 140.42) (width 0.762) (layer F.Cu) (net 4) (status 400000))
 (segment (start 203 128) (end 199.75 124.75) (width 0.762) (layer F.Cu) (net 4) (status 800000))
 (segment (start 203 129.5) (end 203 128) (width 0.762) (layer F.Cu) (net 4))
 (segment (start 192.08 140.42) (end 203 129.5) (width 0.762) (layer F.Cu) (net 4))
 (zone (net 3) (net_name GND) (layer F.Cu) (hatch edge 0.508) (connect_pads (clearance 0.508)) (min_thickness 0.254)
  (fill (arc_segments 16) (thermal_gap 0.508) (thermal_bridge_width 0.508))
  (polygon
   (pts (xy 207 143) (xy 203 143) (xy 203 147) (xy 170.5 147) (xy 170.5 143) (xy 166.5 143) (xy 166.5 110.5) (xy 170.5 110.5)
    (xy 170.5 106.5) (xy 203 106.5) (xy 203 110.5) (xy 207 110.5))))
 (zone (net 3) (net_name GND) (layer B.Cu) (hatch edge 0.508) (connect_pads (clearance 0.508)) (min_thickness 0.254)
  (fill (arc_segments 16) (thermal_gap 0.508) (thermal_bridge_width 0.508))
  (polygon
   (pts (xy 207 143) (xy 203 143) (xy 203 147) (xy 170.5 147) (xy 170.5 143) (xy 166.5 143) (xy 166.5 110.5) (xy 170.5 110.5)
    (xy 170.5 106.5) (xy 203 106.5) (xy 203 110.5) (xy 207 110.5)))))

